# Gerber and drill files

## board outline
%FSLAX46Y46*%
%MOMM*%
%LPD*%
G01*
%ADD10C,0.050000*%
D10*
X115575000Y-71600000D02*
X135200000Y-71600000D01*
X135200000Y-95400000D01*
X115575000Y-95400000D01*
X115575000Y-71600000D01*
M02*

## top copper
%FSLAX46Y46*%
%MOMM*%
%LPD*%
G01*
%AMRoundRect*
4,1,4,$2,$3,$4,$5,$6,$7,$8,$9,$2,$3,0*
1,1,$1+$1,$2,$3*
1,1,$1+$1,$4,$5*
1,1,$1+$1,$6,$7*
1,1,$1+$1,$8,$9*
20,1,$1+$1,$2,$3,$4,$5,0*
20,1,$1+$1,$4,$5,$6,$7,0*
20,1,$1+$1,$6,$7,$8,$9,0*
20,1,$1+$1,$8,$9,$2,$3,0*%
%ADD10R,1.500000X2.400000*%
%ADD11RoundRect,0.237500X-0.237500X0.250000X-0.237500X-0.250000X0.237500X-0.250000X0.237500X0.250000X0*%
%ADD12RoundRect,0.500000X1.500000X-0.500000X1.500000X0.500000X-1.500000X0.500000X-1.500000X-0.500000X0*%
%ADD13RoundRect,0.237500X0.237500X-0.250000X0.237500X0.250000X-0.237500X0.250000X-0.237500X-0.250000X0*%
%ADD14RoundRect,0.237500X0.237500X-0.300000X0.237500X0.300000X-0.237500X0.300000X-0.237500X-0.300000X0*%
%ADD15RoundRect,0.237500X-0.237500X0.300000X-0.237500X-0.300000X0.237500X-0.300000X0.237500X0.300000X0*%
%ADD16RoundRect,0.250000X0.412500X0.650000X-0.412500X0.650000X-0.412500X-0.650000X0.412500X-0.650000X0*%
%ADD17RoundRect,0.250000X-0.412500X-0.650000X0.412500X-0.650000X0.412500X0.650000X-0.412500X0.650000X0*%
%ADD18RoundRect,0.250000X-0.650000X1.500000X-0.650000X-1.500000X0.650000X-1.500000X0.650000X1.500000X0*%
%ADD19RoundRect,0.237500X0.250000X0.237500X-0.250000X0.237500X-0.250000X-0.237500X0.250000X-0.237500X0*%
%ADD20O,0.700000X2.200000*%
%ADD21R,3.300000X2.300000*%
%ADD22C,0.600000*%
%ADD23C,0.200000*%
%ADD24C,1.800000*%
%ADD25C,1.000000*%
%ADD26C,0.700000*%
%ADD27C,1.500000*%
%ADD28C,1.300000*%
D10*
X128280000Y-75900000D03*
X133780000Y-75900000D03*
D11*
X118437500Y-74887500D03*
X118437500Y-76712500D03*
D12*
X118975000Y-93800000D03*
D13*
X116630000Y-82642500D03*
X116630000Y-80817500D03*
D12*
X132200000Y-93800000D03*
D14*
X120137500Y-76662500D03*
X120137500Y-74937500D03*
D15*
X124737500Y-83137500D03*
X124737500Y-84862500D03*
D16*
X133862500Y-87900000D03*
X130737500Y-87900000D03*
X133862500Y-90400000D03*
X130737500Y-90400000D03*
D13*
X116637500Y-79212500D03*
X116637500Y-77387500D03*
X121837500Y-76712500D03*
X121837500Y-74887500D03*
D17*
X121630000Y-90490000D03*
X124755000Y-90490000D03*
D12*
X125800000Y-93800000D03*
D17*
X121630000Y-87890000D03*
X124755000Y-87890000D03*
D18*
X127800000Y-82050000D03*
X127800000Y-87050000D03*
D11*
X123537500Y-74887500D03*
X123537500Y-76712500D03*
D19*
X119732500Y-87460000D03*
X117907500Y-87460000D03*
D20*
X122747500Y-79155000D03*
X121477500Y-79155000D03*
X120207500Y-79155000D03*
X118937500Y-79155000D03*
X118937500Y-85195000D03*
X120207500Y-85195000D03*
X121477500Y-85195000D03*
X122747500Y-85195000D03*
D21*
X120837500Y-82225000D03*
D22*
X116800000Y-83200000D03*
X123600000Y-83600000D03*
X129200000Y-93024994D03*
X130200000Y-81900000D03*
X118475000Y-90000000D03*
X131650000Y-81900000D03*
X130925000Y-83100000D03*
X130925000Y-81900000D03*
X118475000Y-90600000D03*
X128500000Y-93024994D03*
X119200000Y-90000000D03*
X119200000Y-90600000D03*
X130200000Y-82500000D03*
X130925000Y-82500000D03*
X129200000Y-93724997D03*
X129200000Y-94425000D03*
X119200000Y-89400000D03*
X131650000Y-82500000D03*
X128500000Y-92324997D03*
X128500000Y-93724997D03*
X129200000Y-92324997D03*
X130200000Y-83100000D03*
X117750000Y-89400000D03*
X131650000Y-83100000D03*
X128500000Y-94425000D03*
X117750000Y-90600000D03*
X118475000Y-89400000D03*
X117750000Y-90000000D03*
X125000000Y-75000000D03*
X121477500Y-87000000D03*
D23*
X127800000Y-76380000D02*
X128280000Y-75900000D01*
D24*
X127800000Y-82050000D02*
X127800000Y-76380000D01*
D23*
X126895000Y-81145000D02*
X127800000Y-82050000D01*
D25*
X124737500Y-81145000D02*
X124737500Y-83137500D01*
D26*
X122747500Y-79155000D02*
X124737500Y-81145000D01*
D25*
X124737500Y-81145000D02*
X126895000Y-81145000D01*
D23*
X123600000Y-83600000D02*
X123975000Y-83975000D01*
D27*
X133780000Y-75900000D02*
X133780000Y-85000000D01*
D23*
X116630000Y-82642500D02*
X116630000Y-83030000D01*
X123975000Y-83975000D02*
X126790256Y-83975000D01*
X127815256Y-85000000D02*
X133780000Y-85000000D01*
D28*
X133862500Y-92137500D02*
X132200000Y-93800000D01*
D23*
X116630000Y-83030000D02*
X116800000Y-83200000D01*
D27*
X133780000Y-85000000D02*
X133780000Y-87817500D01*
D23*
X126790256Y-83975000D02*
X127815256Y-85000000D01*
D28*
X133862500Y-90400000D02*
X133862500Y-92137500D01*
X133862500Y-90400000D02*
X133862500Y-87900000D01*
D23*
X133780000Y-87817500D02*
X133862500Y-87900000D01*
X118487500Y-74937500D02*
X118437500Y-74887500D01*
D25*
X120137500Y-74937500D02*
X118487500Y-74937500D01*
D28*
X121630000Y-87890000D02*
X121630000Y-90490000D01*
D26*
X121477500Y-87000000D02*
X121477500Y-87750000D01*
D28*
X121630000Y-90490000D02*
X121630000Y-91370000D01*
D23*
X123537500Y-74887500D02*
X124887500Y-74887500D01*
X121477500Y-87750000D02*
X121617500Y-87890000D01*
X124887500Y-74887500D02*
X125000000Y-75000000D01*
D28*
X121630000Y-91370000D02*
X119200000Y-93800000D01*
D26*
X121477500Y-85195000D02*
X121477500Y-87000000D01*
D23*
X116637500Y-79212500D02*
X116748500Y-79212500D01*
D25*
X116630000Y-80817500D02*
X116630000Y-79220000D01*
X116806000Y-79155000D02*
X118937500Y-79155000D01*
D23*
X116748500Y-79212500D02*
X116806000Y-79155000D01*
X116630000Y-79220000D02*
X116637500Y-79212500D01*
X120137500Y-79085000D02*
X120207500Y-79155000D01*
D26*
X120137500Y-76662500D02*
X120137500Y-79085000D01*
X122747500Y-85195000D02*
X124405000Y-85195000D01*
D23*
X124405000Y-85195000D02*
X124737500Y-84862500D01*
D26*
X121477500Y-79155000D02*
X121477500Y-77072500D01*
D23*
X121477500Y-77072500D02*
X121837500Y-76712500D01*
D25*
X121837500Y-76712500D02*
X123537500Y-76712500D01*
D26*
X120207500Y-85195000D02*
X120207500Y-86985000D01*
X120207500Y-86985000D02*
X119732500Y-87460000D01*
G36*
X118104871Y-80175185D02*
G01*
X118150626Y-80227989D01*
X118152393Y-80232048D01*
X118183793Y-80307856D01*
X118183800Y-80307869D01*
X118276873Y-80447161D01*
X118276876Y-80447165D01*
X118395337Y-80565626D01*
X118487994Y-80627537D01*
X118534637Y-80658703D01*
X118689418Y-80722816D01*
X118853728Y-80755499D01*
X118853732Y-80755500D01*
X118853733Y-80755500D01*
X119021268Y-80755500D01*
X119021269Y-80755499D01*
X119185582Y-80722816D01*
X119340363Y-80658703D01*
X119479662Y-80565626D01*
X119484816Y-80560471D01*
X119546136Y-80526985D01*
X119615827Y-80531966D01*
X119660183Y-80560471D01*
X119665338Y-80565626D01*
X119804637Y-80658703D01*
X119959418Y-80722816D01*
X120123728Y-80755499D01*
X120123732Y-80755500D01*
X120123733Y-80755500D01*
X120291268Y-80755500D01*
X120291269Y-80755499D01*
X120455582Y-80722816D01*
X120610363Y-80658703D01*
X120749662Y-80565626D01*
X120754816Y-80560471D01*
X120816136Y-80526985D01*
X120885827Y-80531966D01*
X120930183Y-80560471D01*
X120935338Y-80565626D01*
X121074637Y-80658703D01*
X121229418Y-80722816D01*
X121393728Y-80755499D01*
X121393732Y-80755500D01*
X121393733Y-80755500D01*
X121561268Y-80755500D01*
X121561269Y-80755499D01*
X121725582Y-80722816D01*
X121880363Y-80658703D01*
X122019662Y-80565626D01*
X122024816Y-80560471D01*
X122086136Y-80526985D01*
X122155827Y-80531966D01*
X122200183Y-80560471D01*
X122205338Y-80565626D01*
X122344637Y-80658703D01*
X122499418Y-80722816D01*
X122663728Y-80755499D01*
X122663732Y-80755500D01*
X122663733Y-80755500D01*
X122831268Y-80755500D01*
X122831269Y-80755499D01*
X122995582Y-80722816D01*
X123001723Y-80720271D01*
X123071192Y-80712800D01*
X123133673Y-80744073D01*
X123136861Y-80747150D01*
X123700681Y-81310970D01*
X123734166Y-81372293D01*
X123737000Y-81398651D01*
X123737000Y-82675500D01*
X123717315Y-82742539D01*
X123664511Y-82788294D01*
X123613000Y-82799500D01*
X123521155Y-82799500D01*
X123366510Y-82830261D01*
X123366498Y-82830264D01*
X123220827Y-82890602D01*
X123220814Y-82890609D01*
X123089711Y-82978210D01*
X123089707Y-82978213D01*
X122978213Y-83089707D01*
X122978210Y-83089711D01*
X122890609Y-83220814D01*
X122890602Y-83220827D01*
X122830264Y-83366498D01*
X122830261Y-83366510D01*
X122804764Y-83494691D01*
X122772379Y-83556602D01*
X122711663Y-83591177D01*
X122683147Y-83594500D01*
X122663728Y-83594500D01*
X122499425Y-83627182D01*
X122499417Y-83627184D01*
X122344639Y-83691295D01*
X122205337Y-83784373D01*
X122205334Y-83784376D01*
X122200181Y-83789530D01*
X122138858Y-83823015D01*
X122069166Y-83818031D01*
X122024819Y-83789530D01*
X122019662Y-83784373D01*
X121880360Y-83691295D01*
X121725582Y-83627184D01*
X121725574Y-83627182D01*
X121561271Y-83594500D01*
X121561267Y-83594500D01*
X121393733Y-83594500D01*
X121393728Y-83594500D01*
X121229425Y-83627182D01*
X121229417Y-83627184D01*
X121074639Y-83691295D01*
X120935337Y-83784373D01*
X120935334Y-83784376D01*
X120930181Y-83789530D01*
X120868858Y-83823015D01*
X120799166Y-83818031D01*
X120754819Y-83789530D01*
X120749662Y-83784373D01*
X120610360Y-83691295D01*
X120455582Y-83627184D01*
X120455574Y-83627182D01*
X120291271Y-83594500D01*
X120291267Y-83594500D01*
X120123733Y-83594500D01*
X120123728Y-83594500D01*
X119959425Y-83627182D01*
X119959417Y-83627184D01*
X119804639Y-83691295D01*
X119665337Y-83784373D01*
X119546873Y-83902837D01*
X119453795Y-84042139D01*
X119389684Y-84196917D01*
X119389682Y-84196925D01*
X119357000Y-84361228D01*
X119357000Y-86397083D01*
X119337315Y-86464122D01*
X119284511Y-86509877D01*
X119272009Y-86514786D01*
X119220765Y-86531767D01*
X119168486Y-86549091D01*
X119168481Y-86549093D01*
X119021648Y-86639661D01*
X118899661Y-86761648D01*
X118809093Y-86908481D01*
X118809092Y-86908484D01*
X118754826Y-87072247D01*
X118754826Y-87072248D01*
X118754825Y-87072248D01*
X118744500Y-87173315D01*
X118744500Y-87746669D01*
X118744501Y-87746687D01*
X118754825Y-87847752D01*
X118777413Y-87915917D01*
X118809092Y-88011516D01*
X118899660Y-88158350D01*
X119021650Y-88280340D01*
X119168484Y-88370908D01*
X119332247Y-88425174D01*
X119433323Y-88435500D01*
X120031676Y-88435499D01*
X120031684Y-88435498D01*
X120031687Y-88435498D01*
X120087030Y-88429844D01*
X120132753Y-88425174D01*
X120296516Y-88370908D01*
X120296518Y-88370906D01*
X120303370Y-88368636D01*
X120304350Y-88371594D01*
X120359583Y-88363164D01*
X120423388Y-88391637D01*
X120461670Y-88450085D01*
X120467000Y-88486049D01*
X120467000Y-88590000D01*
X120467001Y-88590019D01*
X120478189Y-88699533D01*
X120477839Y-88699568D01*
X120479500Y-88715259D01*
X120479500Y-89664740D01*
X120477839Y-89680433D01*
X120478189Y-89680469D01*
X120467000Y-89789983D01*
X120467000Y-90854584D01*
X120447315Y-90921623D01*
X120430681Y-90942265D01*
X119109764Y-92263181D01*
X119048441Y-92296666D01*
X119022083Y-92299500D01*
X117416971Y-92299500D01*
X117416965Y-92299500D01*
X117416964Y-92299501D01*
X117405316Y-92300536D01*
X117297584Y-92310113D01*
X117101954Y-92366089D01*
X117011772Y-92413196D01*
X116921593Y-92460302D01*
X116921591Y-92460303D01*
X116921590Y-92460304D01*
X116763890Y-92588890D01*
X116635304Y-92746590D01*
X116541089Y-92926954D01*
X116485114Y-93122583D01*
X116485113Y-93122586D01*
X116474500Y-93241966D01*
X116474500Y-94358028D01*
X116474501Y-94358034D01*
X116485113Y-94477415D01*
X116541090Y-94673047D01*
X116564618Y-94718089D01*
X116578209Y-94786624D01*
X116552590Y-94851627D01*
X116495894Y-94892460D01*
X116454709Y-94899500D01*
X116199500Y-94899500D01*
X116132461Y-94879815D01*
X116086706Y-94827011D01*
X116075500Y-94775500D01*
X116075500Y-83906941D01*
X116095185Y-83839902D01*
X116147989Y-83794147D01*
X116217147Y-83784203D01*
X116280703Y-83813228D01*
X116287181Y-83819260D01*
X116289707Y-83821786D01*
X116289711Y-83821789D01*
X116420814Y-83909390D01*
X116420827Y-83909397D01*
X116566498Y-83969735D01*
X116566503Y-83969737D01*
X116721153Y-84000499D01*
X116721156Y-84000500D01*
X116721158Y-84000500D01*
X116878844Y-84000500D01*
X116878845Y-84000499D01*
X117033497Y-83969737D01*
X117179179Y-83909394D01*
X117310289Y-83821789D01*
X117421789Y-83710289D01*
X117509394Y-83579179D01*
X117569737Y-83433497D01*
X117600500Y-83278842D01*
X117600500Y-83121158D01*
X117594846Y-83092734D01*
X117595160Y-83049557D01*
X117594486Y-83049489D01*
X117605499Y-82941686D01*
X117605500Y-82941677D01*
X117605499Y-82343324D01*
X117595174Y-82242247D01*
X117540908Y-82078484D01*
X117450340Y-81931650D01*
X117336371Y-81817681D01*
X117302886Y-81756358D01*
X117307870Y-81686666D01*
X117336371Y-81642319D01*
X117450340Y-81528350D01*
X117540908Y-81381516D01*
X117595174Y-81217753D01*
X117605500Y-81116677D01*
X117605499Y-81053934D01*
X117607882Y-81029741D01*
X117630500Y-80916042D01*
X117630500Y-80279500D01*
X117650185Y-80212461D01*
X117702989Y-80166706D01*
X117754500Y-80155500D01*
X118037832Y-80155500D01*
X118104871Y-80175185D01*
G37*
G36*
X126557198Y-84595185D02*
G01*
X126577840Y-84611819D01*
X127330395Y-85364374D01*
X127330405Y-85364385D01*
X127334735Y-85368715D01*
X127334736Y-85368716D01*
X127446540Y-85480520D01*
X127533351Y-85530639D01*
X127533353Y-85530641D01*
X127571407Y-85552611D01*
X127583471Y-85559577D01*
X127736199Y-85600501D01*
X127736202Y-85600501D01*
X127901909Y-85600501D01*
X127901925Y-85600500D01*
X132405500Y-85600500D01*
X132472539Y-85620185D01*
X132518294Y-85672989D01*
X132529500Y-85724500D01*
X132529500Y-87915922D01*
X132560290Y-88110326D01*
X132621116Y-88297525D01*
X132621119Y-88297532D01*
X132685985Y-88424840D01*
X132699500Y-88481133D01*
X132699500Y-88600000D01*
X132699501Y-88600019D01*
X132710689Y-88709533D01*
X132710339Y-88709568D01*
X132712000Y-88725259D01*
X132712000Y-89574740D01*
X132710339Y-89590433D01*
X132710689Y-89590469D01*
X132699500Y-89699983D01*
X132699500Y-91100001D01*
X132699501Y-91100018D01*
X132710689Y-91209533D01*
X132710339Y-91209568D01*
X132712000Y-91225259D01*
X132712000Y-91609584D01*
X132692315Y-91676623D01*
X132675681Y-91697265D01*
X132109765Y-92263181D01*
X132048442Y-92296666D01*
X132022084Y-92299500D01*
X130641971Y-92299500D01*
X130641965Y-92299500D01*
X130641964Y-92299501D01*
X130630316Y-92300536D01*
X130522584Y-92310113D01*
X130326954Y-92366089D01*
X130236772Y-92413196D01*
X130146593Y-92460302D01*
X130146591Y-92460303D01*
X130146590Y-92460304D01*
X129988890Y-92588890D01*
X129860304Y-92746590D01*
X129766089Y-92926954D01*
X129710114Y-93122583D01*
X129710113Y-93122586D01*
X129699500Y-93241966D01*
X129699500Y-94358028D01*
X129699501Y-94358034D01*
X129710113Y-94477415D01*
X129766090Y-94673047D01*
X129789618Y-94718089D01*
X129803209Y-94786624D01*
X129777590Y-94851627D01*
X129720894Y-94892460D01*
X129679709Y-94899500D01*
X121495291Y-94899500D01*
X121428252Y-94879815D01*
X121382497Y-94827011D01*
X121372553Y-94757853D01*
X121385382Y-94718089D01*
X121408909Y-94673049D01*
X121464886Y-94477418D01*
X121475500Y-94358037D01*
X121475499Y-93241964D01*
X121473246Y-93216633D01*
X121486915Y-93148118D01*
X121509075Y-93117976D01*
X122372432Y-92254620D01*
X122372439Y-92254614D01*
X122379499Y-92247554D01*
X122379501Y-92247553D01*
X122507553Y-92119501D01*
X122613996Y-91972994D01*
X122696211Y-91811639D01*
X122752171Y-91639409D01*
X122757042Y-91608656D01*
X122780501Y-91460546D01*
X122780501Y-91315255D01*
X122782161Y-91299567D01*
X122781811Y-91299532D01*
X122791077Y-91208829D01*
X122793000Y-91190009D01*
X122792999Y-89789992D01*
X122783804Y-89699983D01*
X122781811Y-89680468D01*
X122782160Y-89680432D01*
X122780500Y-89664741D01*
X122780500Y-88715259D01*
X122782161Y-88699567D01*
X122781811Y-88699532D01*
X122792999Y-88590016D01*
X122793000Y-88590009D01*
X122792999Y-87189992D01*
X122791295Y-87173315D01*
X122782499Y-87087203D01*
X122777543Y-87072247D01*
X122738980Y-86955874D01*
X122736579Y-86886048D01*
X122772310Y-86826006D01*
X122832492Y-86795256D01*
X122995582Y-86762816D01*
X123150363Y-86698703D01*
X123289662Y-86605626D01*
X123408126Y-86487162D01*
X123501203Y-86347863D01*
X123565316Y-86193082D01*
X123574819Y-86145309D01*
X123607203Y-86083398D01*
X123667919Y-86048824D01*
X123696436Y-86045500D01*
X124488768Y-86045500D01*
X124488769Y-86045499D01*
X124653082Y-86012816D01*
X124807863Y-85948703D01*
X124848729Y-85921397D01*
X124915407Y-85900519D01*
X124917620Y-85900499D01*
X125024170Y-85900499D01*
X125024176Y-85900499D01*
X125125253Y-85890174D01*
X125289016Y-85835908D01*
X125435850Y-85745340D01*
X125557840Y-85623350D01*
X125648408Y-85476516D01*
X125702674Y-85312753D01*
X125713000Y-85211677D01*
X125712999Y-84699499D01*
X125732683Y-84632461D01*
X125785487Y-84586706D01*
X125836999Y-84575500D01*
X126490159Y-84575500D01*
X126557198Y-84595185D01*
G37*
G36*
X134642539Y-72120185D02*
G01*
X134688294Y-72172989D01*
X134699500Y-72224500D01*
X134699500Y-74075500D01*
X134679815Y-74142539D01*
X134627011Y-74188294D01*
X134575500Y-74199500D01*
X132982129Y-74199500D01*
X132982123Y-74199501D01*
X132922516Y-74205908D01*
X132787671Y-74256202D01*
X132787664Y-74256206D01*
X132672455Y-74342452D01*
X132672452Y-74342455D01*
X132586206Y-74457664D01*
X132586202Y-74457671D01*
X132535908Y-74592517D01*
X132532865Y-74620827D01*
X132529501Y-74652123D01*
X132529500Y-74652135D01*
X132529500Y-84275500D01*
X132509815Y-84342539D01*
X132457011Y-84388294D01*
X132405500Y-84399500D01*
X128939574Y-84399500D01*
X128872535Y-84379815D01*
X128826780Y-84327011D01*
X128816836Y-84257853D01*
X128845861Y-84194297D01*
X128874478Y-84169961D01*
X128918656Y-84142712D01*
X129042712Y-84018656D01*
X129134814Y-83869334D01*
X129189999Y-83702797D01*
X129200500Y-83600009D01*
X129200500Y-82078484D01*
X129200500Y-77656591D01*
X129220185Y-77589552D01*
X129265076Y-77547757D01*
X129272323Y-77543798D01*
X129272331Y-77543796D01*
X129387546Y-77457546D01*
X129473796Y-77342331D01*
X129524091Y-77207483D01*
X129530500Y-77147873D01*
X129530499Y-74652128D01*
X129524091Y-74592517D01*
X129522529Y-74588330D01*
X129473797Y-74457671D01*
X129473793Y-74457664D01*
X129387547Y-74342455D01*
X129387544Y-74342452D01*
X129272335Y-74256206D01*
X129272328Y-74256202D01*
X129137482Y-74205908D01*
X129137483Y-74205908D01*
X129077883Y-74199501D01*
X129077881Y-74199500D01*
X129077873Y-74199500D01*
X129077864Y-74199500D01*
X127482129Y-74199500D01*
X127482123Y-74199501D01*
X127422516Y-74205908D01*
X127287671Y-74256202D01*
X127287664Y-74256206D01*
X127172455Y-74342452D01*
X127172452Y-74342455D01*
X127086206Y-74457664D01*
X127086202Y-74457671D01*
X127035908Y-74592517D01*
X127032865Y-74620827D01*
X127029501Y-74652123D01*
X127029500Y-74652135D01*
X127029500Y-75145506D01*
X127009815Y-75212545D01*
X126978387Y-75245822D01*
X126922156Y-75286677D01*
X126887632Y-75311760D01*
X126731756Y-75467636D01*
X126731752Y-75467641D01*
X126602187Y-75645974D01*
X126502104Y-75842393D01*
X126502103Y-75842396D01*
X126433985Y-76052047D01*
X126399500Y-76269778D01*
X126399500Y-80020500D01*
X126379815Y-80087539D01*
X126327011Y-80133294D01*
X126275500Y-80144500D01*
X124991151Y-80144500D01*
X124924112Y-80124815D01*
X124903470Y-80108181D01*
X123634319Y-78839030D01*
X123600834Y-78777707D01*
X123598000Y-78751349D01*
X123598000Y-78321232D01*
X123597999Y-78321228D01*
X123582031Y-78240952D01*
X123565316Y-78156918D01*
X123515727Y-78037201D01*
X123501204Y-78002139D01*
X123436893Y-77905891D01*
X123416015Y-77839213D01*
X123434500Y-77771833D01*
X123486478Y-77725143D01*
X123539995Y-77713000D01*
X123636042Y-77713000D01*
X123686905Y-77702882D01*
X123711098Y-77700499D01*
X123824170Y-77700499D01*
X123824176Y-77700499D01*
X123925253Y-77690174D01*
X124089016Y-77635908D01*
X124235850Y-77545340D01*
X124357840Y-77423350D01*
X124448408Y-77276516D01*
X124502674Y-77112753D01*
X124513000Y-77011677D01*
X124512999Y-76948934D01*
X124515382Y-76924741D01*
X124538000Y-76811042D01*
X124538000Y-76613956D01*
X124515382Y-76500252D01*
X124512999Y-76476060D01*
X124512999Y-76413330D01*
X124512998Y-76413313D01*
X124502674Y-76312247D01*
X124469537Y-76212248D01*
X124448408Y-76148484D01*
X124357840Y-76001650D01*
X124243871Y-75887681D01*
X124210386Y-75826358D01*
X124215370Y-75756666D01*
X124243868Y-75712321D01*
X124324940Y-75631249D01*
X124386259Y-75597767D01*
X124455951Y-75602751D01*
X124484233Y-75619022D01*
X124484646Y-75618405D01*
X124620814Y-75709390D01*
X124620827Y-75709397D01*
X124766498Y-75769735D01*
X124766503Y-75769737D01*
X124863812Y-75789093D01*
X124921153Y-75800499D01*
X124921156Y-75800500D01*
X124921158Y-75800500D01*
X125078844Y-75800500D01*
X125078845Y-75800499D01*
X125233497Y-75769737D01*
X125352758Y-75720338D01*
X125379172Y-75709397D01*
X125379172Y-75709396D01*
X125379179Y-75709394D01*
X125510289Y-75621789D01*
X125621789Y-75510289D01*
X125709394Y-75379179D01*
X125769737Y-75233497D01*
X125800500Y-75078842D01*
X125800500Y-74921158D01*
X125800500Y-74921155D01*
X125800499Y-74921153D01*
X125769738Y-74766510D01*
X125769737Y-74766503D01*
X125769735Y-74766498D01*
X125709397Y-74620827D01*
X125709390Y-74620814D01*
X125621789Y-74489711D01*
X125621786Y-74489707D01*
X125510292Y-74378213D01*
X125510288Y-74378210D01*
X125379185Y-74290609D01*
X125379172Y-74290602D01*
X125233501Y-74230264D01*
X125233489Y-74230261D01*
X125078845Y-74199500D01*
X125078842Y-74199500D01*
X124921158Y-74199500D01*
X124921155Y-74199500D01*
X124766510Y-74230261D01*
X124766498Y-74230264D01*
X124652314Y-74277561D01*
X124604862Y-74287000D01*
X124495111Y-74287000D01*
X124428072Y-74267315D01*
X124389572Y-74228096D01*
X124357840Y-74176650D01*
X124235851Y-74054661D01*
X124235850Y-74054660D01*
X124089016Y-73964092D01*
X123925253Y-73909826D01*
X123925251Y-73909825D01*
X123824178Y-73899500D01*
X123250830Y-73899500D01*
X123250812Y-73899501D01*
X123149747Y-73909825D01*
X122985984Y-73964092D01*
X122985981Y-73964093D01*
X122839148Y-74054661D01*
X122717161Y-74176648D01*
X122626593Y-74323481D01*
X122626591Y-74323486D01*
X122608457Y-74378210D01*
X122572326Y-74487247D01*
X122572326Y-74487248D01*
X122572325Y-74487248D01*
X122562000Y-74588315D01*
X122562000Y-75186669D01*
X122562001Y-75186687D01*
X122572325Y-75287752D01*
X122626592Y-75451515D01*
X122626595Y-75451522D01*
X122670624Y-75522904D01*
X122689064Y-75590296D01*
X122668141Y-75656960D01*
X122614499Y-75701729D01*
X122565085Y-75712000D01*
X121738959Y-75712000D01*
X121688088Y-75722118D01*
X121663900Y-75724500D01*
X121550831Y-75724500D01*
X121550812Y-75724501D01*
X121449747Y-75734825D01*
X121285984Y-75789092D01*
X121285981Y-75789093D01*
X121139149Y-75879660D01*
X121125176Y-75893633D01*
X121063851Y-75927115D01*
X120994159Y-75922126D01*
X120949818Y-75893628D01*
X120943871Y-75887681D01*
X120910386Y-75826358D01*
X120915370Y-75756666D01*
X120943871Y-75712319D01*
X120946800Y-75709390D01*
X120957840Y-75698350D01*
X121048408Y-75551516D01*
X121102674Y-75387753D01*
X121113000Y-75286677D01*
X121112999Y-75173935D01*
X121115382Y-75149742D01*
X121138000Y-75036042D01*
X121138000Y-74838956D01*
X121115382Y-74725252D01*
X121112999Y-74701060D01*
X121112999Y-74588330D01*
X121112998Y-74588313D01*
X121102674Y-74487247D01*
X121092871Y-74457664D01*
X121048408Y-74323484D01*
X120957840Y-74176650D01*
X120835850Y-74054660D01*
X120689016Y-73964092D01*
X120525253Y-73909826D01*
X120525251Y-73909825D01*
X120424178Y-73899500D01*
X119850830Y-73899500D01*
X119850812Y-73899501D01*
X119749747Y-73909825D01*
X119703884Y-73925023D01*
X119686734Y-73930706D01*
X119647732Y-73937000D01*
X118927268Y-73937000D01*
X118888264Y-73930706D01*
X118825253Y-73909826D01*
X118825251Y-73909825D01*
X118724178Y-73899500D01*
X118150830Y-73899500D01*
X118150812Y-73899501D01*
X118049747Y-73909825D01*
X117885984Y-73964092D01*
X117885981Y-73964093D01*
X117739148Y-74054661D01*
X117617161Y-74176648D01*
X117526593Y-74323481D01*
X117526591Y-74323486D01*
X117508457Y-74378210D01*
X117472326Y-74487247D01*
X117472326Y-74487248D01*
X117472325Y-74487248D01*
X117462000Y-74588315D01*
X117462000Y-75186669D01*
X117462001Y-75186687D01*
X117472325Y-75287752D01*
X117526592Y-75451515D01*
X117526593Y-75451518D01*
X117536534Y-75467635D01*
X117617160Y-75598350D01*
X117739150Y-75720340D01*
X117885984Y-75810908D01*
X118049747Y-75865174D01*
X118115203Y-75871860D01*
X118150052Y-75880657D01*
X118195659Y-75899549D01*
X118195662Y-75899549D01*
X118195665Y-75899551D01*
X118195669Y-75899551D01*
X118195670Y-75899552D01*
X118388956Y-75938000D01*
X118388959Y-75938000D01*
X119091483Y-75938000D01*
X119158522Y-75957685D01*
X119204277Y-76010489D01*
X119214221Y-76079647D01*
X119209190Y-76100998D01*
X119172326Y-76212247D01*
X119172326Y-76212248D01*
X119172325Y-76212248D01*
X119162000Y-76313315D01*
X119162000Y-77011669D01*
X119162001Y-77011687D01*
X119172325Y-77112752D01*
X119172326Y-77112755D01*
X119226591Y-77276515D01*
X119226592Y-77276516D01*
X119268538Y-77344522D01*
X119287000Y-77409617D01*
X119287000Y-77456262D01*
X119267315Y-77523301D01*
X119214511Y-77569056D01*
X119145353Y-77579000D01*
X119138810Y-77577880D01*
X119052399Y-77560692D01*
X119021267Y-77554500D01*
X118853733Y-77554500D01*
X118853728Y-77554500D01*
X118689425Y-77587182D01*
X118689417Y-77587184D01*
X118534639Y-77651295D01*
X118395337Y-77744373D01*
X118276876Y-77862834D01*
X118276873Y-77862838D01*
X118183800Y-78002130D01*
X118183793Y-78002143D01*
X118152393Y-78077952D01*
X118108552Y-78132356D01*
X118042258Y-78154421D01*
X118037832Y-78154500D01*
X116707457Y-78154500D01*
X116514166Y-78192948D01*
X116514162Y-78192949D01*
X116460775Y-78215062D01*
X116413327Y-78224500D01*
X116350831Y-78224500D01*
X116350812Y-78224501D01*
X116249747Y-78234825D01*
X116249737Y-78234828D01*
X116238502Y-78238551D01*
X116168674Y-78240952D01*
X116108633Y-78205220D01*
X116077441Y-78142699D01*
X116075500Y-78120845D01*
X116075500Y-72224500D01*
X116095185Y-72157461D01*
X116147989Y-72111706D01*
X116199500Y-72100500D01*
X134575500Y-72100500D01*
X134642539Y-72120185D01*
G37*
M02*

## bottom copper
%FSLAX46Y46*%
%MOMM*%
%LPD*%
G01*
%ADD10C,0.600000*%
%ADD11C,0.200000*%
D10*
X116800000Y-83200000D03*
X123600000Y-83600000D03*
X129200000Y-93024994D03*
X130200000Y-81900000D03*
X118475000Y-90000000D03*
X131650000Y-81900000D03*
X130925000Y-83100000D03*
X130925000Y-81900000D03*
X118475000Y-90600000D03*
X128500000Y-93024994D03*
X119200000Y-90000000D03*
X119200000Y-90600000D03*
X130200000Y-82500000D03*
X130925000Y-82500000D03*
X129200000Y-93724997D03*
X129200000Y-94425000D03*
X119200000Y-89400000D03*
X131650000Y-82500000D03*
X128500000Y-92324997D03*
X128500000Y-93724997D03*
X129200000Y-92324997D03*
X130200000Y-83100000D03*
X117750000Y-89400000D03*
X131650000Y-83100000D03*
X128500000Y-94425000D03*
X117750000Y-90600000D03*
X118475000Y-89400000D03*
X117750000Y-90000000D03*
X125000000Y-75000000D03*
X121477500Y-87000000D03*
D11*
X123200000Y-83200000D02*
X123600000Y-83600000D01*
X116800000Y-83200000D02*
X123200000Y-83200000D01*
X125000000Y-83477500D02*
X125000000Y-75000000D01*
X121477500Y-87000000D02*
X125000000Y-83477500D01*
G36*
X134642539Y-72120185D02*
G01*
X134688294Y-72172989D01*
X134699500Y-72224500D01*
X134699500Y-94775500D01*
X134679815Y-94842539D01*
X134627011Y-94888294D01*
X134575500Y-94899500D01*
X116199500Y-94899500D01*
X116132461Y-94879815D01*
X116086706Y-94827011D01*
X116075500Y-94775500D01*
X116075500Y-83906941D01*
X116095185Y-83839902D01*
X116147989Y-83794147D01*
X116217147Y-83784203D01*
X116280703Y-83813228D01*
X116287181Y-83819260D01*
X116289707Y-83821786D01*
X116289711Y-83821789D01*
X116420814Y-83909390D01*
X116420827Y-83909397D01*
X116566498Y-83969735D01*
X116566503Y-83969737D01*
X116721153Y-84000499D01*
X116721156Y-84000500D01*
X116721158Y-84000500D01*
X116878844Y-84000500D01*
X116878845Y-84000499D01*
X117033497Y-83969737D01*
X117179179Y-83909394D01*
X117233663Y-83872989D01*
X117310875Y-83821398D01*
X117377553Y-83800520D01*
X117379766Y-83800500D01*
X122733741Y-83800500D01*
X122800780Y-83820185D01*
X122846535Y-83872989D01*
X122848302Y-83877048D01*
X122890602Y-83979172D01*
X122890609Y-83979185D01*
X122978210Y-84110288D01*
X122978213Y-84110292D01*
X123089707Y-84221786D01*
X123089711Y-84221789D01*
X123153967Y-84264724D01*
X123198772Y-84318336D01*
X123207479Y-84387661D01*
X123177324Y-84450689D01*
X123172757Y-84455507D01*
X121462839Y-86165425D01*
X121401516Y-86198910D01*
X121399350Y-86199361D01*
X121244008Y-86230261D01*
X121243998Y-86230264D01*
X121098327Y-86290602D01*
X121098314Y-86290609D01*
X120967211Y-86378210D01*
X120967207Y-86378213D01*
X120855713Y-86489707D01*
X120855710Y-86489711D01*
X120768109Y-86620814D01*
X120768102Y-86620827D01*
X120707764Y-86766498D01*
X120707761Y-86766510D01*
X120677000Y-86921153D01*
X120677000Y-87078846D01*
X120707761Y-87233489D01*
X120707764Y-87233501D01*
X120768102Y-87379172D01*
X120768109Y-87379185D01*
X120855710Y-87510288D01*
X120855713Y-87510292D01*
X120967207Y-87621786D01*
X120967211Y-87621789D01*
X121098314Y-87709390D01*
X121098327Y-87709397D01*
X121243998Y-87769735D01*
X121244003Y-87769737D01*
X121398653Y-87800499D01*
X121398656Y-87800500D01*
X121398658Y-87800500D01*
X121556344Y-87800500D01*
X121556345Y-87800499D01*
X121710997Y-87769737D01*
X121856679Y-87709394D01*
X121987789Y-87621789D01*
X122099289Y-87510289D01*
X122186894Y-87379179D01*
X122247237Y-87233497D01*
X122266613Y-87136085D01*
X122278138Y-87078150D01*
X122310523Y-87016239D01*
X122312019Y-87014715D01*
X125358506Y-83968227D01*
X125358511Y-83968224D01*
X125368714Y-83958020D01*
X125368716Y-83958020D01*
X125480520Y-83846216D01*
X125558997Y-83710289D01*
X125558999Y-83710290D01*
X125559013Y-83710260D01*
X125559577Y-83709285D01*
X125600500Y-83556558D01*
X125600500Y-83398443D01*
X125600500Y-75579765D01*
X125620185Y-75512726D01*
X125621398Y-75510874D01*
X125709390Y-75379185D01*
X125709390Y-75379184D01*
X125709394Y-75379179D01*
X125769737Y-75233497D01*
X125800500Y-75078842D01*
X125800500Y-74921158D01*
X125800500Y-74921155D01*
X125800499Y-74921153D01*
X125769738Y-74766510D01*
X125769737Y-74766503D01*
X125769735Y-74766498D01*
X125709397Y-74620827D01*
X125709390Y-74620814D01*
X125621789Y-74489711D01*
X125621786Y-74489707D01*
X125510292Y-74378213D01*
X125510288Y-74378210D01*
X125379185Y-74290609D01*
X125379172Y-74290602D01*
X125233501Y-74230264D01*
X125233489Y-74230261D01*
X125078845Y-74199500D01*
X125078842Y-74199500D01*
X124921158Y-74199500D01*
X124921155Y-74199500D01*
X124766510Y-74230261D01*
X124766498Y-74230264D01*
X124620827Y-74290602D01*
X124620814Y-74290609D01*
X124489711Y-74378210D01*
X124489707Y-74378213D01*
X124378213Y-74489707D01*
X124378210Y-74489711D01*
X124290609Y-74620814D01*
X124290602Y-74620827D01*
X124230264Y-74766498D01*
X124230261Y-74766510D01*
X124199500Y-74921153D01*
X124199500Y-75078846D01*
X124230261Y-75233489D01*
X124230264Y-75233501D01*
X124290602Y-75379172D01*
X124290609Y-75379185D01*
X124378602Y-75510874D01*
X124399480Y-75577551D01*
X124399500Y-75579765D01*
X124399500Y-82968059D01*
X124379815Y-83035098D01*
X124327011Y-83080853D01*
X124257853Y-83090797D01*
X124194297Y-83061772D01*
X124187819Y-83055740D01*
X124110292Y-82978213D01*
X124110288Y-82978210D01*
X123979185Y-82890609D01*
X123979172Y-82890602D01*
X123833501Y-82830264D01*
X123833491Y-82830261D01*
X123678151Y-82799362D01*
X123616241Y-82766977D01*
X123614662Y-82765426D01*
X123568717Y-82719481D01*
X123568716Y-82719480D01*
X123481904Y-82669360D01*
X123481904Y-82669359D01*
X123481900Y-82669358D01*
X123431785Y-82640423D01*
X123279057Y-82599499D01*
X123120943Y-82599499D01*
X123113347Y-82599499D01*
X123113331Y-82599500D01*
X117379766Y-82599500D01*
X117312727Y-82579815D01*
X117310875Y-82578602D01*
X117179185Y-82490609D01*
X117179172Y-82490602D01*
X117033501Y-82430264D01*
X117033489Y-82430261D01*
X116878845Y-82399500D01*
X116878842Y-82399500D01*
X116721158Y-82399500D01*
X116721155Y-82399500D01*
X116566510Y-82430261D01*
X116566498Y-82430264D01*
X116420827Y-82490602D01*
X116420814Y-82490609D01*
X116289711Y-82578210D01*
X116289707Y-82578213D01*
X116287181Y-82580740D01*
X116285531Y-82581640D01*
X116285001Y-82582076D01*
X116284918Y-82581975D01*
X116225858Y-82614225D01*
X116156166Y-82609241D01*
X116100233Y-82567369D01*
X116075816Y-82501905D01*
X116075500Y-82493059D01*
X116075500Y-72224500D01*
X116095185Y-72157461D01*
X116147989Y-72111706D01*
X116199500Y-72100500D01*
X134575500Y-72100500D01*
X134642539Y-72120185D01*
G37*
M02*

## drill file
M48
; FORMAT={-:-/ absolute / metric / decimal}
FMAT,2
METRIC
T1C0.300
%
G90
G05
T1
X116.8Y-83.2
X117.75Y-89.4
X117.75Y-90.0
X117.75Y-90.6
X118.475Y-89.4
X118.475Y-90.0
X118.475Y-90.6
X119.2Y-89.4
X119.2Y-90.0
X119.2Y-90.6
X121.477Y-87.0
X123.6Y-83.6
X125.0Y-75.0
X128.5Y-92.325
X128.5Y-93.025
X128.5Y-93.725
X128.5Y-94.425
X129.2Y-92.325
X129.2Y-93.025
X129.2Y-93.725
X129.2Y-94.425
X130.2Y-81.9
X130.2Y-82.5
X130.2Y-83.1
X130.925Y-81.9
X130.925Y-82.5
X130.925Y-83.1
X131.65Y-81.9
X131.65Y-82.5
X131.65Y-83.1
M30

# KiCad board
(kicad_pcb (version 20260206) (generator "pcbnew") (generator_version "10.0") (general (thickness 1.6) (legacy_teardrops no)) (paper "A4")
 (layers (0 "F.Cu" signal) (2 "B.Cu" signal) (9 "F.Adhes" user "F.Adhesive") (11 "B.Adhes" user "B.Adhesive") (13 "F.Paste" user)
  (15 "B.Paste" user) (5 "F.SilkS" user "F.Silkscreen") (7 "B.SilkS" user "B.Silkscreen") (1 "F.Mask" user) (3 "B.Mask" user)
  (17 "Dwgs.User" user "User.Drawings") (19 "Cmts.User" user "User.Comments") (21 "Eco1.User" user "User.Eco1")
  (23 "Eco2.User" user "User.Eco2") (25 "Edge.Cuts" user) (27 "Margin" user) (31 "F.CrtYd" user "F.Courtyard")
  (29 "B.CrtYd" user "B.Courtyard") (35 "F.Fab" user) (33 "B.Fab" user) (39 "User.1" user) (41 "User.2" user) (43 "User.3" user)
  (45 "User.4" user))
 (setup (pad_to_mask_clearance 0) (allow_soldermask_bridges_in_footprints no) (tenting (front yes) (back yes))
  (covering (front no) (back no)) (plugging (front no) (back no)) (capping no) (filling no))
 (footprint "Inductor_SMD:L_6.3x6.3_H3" (layer "F.Cu") (at 131.03 75.9)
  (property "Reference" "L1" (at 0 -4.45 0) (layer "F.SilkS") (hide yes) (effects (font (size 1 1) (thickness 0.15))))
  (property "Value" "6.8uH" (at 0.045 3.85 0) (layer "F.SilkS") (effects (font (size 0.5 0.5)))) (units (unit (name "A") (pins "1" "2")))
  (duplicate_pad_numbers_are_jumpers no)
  (pad "1" smd rect (at -2.75 0) (size 1.5 2.4) (layers "F.Cu" "F.Mask" "F.Paste") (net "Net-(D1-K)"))
  (pad "2" smd rect (at 2.75 0) (size 1.5 2.4) (layers "F.Cu" "F.Mask" "F.Paste") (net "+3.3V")))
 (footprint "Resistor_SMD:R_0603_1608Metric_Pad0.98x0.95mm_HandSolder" (layer "F.Cu") (at 118.4375 75.8 -90)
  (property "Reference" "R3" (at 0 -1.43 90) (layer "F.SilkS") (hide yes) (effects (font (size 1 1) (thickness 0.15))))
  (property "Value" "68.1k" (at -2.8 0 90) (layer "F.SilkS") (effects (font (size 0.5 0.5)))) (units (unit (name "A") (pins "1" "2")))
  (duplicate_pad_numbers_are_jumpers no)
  (pad "1" smd roundrect (at -0.9125 0 270) (size 0.975 0.95) (layers "F.Cu" "F.Mask" "F.Paste") (roundrect_rratio 0.25)
   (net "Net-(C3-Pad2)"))
  (pad "2" smd roundrect (at 0.9125 0 270) (size 0.975 0.95) (layers "F.Cu" "F.Mask" "F.Paste") (roundrect_rratio 0.25) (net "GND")))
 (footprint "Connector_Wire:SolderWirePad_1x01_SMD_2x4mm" (layer "F.Cu") (at 118.975 93.8 90)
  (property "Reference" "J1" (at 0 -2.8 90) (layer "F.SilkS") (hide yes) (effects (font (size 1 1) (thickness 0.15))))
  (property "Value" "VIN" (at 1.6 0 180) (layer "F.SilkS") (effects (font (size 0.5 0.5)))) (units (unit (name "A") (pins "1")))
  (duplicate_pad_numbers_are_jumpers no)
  (pad "1" smd roundrect (at 0 0 90) (size 2 4) (layers "F.Cu" "F.Mask") (roundrect_rratio 0.25) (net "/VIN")))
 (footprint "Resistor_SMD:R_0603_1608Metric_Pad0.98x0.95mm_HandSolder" (layer "F.Cu") (at 116.63 81.73 90)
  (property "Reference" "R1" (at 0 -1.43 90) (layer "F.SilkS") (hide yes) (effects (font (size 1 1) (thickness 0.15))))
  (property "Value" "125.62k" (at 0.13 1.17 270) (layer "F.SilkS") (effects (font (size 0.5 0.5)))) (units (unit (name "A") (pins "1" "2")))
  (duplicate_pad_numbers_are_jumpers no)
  (pad "1" smd roundrect (at -0.9125 0 90) (size 0.975 0.95) (layers "F.Cu" "F.Mask" "F.Paste") (roundrect_rratio 0.25) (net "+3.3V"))
  (pad "2" smd roundrect (at 0.9125 0 90) (size 0.975 0.95) (layers "F.Cu" "F.Mask" "F.Paste") (roundrect_rratio 0.25)
   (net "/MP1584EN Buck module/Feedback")))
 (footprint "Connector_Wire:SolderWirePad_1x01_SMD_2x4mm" (layer "F.Cu") (at 132.2 93.8 90)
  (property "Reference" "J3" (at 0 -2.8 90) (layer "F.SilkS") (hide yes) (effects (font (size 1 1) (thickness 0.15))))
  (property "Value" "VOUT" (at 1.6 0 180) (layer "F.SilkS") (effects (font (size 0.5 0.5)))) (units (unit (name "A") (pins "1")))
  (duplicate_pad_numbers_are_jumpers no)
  (pad "1" smd roundrect (at 0 0 90) (size 2 4) (layers "F.Cu" "F.Mask") (roundrect_rratio 0.25) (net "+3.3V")))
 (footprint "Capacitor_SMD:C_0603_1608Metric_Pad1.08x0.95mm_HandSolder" (layer "F.Cu") (at 120.1375 75.8 90)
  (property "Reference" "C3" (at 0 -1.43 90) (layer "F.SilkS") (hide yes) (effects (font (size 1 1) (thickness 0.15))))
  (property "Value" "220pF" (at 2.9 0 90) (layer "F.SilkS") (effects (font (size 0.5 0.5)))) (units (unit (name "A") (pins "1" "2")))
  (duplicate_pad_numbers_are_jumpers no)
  (pad "1" smd roundrect (at -0.8625 0 90) (size 1.075 0.95) (layers "F.Cu" "F.Mask" "F.Paste") (roundrect_rratio 0.25)
   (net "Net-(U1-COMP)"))
  (pad "2" smd roundrect (at 0.8625 0 90) (size 1.075 0.95) (layers "F.Cu" "F.Mask" "F.Paste") (roundrect_rratio 0.25) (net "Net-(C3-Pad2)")))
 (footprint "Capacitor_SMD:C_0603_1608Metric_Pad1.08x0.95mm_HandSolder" (layer "F.Cu") (at 124.7375 84 -90)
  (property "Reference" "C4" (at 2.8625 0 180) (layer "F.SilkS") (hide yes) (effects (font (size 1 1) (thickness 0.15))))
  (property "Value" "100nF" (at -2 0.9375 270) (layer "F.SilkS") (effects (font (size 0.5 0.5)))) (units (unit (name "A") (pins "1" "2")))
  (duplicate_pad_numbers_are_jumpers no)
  (pad "1" smd roundrect (at -0.8625 0 270) (size 1.075 0.95) (layers "F.Cu" "F.Mask" "F.Paste") (roundrect_rratio 0.25) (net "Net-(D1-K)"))
  (pad "2" smd roundrect (at 0.8625 0 270) (size 1.075 0.95) (layers "F.Cu" "F.Mask" "F.Paste") (roundrect_rratio 0.25) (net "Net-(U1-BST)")))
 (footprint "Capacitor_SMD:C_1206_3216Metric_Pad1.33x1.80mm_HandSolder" (layer "F.Cu") (at 132.3 87.9 180)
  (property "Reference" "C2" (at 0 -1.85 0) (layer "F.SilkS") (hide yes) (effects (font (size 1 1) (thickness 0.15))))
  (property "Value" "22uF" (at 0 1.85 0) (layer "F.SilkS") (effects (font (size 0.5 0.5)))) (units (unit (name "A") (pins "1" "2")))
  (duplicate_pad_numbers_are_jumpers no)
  (pad "1" smd roundrect (at -1.5625 0 180) (size 1.325 1.8) (layers "F.Cu" "F.Mask" "F.Paste") (roundrect_rratio 0.188679) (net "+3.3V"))
  (pad "2" smd roundrect (at 1.5625 0 180) (size 1.325 1.8) (layers "F.Cu" "F.Mask" "F.Paste") (roundrect_rratio 0.188679) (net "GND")))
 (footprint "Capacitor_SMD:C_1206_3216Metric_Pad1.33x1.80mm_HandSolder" (layer "F.Cu") (at 132.3 90.4 180)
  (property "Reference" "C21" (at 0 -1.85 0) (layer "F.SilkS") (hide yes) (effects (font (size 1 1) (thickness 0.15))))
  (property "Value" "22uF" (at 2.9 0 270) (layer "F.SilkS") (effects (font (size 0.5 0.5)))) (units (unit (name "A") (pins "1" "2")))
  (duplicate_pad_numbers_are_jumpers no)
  (pad "1" smd roundrect (at -1.5625 0 180) (size 1.325 1.8) (layers "F.Cu" "F.Mask" "F.Paste") (roundrect_rratio 0.188679) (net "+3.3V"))
  (pad "2" smd roundrect (at 1.5625 0 180) (size 1.325 1.8) (layers "F.Cu" "F.Mask" "F.Paste") (roundrect_rratio 0.188679) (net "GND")))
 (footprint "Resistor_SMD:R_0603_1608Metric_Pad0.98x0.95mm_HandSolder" (layer "F.Cu") (at 116.6375 78.3 90)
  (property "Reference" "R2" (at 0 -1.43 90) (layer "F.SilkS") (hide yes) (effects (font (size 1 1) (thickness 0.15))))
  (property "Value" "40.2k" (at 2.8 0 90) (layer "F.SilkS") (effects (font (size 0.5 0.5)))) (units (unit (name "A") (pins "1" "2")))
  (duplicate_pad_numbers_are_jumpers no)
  (pad "1" smd roundrect (at -0.9125 0 90) (size 0.975 0.95) (layers "F.Cu" "F.Mask" "F.Paste") (roundrect_rratio 0.25)
   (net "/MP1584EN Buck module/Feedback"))
  (pad "2" smd roundrect (at 0.9125 0 90) (size 0.975 0.95) (layers "F.Cu" "F.Mask" "F.Paste") (roundrect_rratio 0.25) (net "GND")))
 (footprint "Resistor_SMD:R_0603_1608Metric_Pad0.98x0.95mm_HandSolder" (layer "F.Cu") (at 121.8375 75.8 90)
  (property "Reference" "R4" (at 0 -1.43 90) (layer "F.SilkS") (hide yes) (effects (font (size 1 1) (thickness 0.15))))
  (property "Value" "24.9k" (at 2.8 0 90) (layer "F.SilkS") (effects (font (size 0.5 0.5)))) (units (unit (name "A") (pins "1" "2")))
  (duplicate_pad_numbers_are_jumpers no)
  (pad "1" smd roundrect (at -0.9125 0 90) (size 0.975 0.95) (layers "F.Cu" "F.Mask" "F.Paste") (roundrect_rratio 0.25) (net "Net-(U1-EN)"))
  (pad "2" smd roundrect (at 0.9125 0 90) (size 0.975 0.95) (layers "F.Cu" "F.Mask" "F.Paste") (roundrect_rratio 0.25) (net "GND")))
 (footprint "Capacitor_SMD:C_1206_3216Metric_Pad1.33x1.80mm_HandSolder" (layer "F.Cu") (at 123.1925 90.49)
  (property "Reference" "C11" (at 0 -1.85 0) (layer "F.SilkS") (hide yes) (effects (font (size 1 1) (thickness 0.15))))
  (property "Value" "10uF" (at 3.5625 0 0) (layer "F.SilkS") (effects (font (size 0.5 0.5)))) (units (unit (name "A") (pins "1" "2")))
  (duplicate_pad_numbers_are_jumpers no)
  (pad "1" smd roundrect (at -1.5625 0) (size 1.325 1.8) (layers "F.Cu" "F.Mask" "F.Paste") (roundrect_rratio 0.188679) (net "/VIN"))
  (pad "2" smd roundrect (at 1.5625 0) (size 1.325 1.8) (layers "F.Cu" "F.Mask" "F.Paste") (roundrect_rratio 0.188679) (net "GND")))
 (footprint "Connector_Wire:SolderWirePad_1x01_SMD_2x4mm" (layer "F.Cu") (at 125.8 93.8 90)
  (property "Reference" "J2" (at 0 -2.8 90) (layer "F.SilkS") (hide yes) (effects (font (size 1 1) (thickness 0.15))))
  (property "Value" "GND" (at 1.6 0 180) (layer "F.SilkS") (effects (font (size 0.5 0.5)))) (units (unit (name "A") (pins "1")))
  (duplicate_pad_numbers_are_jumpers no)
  (pad "1" smd roundrect (at 0 0 90) (size 2 4) (layers "F.Cu" "F.Mask") (roundrect_rratio 0.25) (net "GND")))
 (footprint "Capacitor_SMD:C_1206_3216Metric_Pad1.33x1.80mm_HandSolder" (layer "F.Cu") (at 123.1925 87.89)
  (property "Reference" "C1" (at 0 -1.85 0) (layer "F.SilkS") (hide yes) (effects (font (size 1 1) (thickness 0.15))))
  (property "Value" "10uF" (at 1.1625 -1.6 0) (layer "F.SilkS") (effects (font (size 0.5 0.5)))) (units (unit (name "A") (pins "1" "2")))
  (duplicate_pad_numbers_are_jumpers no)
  (pad "1" smd roundrect (at -1.5625 0) (size 1.325 1.8) (layers "F.Cu" "F.Mask" "F.Paste") (roundrect_rratio 0.188679) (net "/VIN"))
  (pad "2" smd roundrect (at 1.5625 0) (size 1.325 1.8) (layers "F.Cu" "F.Mask" "F.Paste") (roundrect_rratio 0.188679) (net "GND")))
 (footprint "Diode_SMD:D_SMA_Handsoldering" (layer "F.Cu") (at 127.8 84.55 -90)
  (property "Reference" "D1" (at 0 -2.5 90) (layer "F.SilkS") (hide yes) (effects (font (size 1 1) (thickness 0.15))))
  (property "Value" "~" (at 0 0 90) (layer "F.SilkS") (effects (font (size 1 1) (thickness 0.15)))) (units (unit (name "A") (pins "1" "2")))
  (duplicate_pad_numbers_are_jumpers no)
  (pad "1" smd roundrect (at -2.5 0 270) (size 3.5 1.8) (layers "F.Cu" "F.Mask" "F.Paste") (roundrect_rratio 0.1388888889)
   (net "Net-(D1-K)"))
  (pad "2" smd roundrect (at 2.5 0 270) (size 3.5 1.8) (layers "F.Cu" "F.Mask" "F.Paste") (roundrect_rratio 0.1388888889) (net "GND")))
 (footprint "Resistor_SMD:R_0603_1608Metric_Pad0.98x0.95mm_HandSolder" (layer "F.Cu") (at 123.5375 75.8 -90)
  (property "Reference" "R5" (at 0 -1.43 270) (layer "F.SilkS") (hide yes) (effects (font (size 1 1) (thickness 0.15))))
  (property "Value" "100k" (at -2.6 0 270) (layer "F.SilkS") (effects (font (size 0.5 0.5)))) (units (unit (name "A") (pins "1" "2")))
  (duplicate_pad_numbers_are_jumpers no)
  (pad "1" smd roundrect (at -0.9125 0 270) (size 0.975 0.95) (layers "F.Cu" "F.Mask" "F.Paste") (roundrect_rratio 0.25) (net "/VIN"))
  (pad "2" smd roundrect (at 0.9125 0 270) (size 0.975 0.95) (layers "F.Cu" "F.Mask" "F.Paste") (roundrect_rratio 0.25) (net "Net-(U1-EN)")))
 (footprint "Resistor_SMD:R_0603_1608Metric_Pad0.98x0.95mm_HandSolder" (layer "F.Cu") (at 118.82 87.46 180)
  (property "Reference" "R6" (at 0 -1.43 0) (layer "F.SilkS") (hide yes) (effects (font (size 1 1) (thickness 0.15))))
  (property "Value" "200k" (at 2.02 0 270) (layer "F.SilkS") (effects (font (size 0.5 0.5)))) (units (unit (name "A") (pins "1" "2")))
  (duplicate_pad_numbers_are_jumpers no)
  (pad "1" smd roundrect (at -0.9125 0 180) (size 0.975 0.95) (layers "F.Cu" "F.Mask" "F.Paste") (roundrect_rratio 0.25)
   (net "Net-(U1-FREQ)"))
  (pad "2" smd roundrect (at 0.9125 0 180) (size 0.975 0.95) (layers "F.Cu" "F.Mask" "F.Paste") (roundrect_rratio 0.25) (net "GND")))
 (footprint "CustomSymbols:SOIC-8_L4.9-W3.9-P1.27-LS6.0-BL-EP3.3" (layer "F.Cu") (at 120.8375 82.175 180)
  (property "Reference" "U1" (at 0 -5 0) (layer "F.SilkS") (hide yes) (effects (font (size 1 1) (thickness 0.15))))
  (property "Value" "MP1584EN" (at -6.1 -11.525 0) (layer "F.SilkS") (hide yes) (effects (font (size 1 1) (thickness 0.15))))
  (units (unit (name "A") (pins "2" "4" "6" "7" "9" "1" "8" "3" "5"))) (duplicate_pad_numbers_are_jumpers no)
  (pad "1" smd oval (at -1.91 3.02) (size 0.7 2.2) (layers "F.Cu" "F.Mask" "F.Paste") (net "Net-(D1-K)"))
  (pad "2" smd oval (at -0.64 3.02) (size 0.7 2.2) (layers "F.Cu" "F.Mask" "F.Paste") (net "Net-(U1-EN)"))
  (pad "3" smd oval (at 0.63 3.02) (size 0.7 2.2) (layers "F.Cu" "F.Mask" "F.Paste") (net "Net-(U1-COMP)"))
  (pad "4" smd oval (at 1.9 3.02) (size 0.7 2.2) (layers "F.Cu" "F.Mask" "F.Paste") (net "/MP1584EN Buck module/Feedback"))
  (pad "5" smd oval (at 1.9 -3.02) (size 0.7 2.2) (layers "F.Cu" "F.Mask" "F.Paste") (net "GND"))
  (pad "6" smd oval (at 0.63 -3.02) (size 0.7 2.2) (layers "F.Cu" "F.Mask" "F.Paste") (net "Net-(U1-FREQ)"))
  (pad "7" smd oval (at -0.64 -3.02) (size 0.7 2.2) (layers "F.Cu" "F.Mask" "F.Paste") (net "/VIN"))
  (pad "8" smd oval (at -1.91 -3.02) (size 0.7 2.2) (layers "F.Cu" "F.Mask" "F.Paste") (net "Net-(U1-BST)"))
  (pad "9" smd rect (at 0 -0.05 270) (size 2.3 3.3) (layers "F.Cu" "F.Mask" "F.Paste") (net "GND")))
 (gr_rect (start 115.575 71.6) (end 135.2 95.4) (stroke (width 0.05) (type default)) (fill no) (layer "Edge.Cuts"))
 (segment (start 127.8 76.38) (end 128.28 75.9) (width 0.2) (layer "F.Cu") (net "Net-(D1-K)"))
 (segment (start 127.8 82.05) (end 127.8 76.38) (width 1.8) (layer "F.Cu") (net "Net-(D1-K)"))
 (segment (start 126.895 81.145) (end 127.8 82.05) (width 0.2) (layer "F.Cu") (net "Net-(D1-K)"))
 (segment (start 124.7375 81.145) (end 124.7375 83.1375) (width 1) (layer "F.Cu") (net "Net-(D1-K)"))
 (segment (start 122.7475 79.155) (end 124.7375 81.145) (width 0.7) (layer "F.Cu") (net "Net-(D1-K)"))
 (segment (start 124.7375 81.145) (end 126.895 81.145) (width 1) (layer "F.Cu") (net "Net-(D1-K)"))
 (segment (start 123.6 83.6) (end 123.975 83.975) (width 0.2) (layer "F.Cu") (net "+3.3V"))
 (segment (start 133.78 75.9) (end 133.78 85) (width 1.5) (layer "F.Cu") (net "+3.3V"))
 (segment (start 116.63 82.6425) (end 116.63 83.03) (width 0.2) (layer "F.Cu") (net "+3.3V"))
 (segment (start 123.975 83.975) (end 126.790256 83.975) (width 0.2) (layer "F.Cu") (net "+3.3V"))
 (segment (start 127.815256 85) (end 133.78 85) (width 0.2) (layer "F.Cu") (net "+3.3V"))
 (segment (start 133.8625 92.1375) (end 132.2 93.8) (width 1.3) (layer "F.Cu") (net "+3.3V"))
 (segment (start 116.63 83.03) (end 116.8 83.2) (width 0.2) (layer "F.Cu") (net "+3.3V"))
 (segment (start 133.78 85) (end 133.78 87.8175) (width 1.5) (layer "F.Cu") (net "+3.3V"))
 (segment (start 126.790256 83.975) (end 127.815256 85) (width 0.2) (layer "F.Cu") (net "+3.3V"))
 (segment (start 133.8625 90.4) (end 133.8625 92.1375) (width 1.3) (layer "F.Cu") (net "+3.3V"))
 (segment (start 133.8625 90.4) (end 133.8625 87.9) (width 1.3) (layer "F.Cu") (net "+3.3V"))
 (segment (start 133.78 87.8175) (end 133.8625 87.9) (width 0.2) (layer "F.Cu") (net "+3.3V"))
 (via (at 116.8 83.2) (size 0.6) (drill 0.3) (layers "F.Cu" "B.Cu") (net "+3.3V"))
 (via (at 123.6 83.6) (size 0.6) (drill 0.3) (layers "F.Cu" "B.Cu") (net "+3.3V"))
 (segment (start 123.2 83.2) (end 123.6 83.6) (width 0.2) (layer "B.Cu") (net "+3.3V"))
 (segment (start 116.8 83.2) (end 123.2 83.2) (width 0.2) (layer "B.Cu") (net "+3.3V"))
 (segment (start 118.4875 74.9375) (end 118.4375 74.8875) (width 0.2) (layer "F.Cu") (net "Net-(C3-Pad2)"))
 (segment (start 120.1375 74.9375) (end 118.4875 74.9375) (width 1) (layer "F.Cu") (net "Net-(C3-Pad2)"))
 (via (at 129.2 93.024994) (size 0.6) (drill 0.3) (layers "F.Cu" "B.Cu") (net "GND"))
 (via (at 130.2 81.9) (size 0.6) (drill 0.3) (layers "F.Cu" "B.Cu") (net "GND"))
 (via (at 118.475 90) (size 0.6) (drill 0.3) (layers "F.Cu" "B.Cu") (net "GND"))
 (via (at 131.65 81.9) (size 0.6) (drill 0.3) (layers "F.Cu" "B.Cu") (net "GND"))
 (via (at 130.925 83.1) (size 0.6) (drill 0.3) (layers "F.Cu" "B.Cu") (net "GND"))
 (via (at 130.925 81.9) (size 0.6) (drill 0.3) (layers "F.Cu" "B.Cu") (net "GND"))
 (via (at 118.475 90.6) (size 0.6) (drill 0.3) (layers "F.Cu" "B.Cu") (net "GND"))
 (via (at 128.5 93.024994) (size 0.6) (drill 0.3) (layers "F.Cu" "B.Cu") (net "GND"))
 (via (at 119.2 90) (size 0.6) (drill 0.3) (layers "F.Cu" "B.Cu") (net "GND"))
 (via (at 119.2 90.6) (size 0.6) (drill 0.3) (layers "F.Cu" "B.Cu") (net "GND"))
 (via (at 130.2 82.5) (size 0.6) (drill 0.3) (layers "F.Cu" "B.Cu") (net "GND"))
 (via (at 130.925 82.5) (size 0.6) (drill 0.3) (layers "F.Cu" "B.Cu") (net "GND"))
 (via (at 129.2 93.724997) (size 0.6) (drill 0.3) (layers "F.Cu" "B.Cu") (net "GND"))
 (via (at 129.2 94.425) (size 0.6) (drill 0.3) (layers "F.Cu" "B.Cu") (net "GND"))
 (via (at 119.2 89.4) (size 0.6) (drill 0.3) (layers "F.Cu" "B.Cu") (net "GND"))
 (via (at 131.65 82.5) (size 0.6) (drill 0.3) (layers "F.Cu" "B.Cu") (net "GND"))
 (via (at 128.5 92.324997) (size 0.6) (drill 0.3) (layers "F.Cu" "B.Cu") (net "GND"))
 (via (at 128.5 93.724997) (size 0.6) (drill 0.3) (layers "F.Cu" "B.Cu") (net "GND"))
 (via (at 129.2 92.324997) (size 0.6) (drill 0.3) (layers "F.Cu" "B.Cu") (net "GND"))
 (via (at 130.2 83.1) (size 0.6) (drill 0.3) (layers "F.Cu" "B.Cu") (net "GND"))
 (via (at 117.75 89.4) (size 0.6) (drill 0.3) (layers "F.Cu" "B.Cu") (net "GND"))
 (via (at 131.65 83.1) (size 0.6) (drill 0.3) (layers "F.Cu" "B.Cu") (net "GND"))
 (via (at 128.5 94.425) (size 0.6) (drill 0.3) (layers "F.Cu" "B.Cu") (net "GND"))
 (via (at 117.75 90.6) (size 0.6) (drill 0.3) (layers "F.Cu" "B.Cu") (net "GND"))
 (via (at 118.475 89.4) (size 0.6) (drill 0.3) (layers "F.Cu" "B.Cu") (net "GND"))
 (via (at 117.75 90) (size 0.6) (drill 0.3) (layers "F.Cu" "B.Cu") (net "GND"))
 (segment (start 121.63 87.89) (end 121.63 90.49) (width 1.3) (layer "F.Cu") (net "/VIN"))
 (segment (start 121.4775 87) (end 121.4775 87.75) (width 0.7) (layer "F.Cu") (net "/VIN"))
 (segment (start 121.63 90.49) (end 121.63 91.37) (width 1.3) (layer "F.Cu") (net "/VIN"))
 (segment (start 123.5375 74.8875) (end 124.8875 74.8875) (width 0.2) (layer "F.Cu") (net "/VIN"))
 (segment (start 121.4775 87.75) (end 121.6175 87.89) (width 0.2) (layer "F.Cu") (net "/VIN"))
 (segment (start 124.8875 74.8875) (end 125 75) (width 0.2) (layer "F.Cu") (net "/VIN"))
 (segment (start 121.63 91.37) (end 119.2 93.8) (width 1.3) (layer "F.Cu") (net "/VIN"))
 (segment (start 121.4775 85.195) (end 121.4775 87) (width 0.7) (layer "F.Cu") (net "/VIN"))
 (via (at 125 75) (size 0.6) (drill 0.3) (layers "F.Cu" "B.Cu") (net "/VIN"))
 (via (at 121.4775 87) (size 0.6) (drill 0.3) (layers "F.Cu" "B.Cu") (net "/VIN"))
 (segment (start 125 83.4775) (end 125 75) (width 0.2) (layer "B.Cu") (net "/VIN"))
 (segment (start 121.4775 87) (end 125 83.4775) (width 0.2) (layer "B.Cu") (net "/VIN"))
 (segment (start 116.6375 79.2125) (end 116.7485 79.2125) (width 0.2) (layer "F.Cu") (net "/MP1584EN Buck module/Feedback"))
 (segment (start 116.63 80.8175) (end 116.63 79.22) (width 1) (layer "F.Cu") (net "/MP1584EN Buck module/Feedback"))
 (segment (start 116.806 79.155) (end 118.9375 79.155) (width 1) (layer "F.Cu") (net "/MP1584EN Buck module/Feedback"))
 (segment (start 116.7485 79.2125) (end 116.806 79.155) (width 0.2) (layer "F.Cu") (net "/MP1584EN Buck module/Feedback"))
 (segment (start 116.63 79.22) (end 116.6375 79.2125) (width 0.2) (layer "F.Cu") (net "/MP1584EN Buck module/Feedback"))
 (segment (start 120.1375 79.085) (end 120.2075 79.155) (width 0.2) (layer "F.Cu") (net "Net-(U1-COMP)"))
 (segment (start 120.1375 76.6625) (end 120.1375 79.085) (width 0.7) (layer "F.Cu") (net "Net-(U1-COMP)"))
 (segment (start 122.7475 85.195) (end 124.405 85.195) (width 0.7) (layer "F.Cu") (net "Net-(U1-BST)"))
 (segment (start 124.405 85.195) (end 124.7375 84.8625) (width 0.2) (layer "F.Cu") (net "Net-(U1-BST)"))
 (segment (start 121.4775 79.155) (end 121.4775 77.0725) (width 0.7) (layer "F.Cu") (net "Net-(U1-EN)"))
 (segment (start 121.4775 77.0725) (end 121.8375 76.7125) (width 0.2) (layer "F.Cu") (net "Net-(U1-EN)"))
 (segment (start 121.8375 76.7125) (end 123.5375 76.7125) (width 1) (layer "F.Cu") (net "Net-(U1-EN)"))
 (segment (start 120.2075 85.195) (end 120.2075 86.985) (width 0.7) (layer "F.Cu") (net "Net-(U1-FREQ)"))
 (segment (start 120.2075 86.985) (end 119.7325 87.46) (width 0.7) (layer "F.Cu") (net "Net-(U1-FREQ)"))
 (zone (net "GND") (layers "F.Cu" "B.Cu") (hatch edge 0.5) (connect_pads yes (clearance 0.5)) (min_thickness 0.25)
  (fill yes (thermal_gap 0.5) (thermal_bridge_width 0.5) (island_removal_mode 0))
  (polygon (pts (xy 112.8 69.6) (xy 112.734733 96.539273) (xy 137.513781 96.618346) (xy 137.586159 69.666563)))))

